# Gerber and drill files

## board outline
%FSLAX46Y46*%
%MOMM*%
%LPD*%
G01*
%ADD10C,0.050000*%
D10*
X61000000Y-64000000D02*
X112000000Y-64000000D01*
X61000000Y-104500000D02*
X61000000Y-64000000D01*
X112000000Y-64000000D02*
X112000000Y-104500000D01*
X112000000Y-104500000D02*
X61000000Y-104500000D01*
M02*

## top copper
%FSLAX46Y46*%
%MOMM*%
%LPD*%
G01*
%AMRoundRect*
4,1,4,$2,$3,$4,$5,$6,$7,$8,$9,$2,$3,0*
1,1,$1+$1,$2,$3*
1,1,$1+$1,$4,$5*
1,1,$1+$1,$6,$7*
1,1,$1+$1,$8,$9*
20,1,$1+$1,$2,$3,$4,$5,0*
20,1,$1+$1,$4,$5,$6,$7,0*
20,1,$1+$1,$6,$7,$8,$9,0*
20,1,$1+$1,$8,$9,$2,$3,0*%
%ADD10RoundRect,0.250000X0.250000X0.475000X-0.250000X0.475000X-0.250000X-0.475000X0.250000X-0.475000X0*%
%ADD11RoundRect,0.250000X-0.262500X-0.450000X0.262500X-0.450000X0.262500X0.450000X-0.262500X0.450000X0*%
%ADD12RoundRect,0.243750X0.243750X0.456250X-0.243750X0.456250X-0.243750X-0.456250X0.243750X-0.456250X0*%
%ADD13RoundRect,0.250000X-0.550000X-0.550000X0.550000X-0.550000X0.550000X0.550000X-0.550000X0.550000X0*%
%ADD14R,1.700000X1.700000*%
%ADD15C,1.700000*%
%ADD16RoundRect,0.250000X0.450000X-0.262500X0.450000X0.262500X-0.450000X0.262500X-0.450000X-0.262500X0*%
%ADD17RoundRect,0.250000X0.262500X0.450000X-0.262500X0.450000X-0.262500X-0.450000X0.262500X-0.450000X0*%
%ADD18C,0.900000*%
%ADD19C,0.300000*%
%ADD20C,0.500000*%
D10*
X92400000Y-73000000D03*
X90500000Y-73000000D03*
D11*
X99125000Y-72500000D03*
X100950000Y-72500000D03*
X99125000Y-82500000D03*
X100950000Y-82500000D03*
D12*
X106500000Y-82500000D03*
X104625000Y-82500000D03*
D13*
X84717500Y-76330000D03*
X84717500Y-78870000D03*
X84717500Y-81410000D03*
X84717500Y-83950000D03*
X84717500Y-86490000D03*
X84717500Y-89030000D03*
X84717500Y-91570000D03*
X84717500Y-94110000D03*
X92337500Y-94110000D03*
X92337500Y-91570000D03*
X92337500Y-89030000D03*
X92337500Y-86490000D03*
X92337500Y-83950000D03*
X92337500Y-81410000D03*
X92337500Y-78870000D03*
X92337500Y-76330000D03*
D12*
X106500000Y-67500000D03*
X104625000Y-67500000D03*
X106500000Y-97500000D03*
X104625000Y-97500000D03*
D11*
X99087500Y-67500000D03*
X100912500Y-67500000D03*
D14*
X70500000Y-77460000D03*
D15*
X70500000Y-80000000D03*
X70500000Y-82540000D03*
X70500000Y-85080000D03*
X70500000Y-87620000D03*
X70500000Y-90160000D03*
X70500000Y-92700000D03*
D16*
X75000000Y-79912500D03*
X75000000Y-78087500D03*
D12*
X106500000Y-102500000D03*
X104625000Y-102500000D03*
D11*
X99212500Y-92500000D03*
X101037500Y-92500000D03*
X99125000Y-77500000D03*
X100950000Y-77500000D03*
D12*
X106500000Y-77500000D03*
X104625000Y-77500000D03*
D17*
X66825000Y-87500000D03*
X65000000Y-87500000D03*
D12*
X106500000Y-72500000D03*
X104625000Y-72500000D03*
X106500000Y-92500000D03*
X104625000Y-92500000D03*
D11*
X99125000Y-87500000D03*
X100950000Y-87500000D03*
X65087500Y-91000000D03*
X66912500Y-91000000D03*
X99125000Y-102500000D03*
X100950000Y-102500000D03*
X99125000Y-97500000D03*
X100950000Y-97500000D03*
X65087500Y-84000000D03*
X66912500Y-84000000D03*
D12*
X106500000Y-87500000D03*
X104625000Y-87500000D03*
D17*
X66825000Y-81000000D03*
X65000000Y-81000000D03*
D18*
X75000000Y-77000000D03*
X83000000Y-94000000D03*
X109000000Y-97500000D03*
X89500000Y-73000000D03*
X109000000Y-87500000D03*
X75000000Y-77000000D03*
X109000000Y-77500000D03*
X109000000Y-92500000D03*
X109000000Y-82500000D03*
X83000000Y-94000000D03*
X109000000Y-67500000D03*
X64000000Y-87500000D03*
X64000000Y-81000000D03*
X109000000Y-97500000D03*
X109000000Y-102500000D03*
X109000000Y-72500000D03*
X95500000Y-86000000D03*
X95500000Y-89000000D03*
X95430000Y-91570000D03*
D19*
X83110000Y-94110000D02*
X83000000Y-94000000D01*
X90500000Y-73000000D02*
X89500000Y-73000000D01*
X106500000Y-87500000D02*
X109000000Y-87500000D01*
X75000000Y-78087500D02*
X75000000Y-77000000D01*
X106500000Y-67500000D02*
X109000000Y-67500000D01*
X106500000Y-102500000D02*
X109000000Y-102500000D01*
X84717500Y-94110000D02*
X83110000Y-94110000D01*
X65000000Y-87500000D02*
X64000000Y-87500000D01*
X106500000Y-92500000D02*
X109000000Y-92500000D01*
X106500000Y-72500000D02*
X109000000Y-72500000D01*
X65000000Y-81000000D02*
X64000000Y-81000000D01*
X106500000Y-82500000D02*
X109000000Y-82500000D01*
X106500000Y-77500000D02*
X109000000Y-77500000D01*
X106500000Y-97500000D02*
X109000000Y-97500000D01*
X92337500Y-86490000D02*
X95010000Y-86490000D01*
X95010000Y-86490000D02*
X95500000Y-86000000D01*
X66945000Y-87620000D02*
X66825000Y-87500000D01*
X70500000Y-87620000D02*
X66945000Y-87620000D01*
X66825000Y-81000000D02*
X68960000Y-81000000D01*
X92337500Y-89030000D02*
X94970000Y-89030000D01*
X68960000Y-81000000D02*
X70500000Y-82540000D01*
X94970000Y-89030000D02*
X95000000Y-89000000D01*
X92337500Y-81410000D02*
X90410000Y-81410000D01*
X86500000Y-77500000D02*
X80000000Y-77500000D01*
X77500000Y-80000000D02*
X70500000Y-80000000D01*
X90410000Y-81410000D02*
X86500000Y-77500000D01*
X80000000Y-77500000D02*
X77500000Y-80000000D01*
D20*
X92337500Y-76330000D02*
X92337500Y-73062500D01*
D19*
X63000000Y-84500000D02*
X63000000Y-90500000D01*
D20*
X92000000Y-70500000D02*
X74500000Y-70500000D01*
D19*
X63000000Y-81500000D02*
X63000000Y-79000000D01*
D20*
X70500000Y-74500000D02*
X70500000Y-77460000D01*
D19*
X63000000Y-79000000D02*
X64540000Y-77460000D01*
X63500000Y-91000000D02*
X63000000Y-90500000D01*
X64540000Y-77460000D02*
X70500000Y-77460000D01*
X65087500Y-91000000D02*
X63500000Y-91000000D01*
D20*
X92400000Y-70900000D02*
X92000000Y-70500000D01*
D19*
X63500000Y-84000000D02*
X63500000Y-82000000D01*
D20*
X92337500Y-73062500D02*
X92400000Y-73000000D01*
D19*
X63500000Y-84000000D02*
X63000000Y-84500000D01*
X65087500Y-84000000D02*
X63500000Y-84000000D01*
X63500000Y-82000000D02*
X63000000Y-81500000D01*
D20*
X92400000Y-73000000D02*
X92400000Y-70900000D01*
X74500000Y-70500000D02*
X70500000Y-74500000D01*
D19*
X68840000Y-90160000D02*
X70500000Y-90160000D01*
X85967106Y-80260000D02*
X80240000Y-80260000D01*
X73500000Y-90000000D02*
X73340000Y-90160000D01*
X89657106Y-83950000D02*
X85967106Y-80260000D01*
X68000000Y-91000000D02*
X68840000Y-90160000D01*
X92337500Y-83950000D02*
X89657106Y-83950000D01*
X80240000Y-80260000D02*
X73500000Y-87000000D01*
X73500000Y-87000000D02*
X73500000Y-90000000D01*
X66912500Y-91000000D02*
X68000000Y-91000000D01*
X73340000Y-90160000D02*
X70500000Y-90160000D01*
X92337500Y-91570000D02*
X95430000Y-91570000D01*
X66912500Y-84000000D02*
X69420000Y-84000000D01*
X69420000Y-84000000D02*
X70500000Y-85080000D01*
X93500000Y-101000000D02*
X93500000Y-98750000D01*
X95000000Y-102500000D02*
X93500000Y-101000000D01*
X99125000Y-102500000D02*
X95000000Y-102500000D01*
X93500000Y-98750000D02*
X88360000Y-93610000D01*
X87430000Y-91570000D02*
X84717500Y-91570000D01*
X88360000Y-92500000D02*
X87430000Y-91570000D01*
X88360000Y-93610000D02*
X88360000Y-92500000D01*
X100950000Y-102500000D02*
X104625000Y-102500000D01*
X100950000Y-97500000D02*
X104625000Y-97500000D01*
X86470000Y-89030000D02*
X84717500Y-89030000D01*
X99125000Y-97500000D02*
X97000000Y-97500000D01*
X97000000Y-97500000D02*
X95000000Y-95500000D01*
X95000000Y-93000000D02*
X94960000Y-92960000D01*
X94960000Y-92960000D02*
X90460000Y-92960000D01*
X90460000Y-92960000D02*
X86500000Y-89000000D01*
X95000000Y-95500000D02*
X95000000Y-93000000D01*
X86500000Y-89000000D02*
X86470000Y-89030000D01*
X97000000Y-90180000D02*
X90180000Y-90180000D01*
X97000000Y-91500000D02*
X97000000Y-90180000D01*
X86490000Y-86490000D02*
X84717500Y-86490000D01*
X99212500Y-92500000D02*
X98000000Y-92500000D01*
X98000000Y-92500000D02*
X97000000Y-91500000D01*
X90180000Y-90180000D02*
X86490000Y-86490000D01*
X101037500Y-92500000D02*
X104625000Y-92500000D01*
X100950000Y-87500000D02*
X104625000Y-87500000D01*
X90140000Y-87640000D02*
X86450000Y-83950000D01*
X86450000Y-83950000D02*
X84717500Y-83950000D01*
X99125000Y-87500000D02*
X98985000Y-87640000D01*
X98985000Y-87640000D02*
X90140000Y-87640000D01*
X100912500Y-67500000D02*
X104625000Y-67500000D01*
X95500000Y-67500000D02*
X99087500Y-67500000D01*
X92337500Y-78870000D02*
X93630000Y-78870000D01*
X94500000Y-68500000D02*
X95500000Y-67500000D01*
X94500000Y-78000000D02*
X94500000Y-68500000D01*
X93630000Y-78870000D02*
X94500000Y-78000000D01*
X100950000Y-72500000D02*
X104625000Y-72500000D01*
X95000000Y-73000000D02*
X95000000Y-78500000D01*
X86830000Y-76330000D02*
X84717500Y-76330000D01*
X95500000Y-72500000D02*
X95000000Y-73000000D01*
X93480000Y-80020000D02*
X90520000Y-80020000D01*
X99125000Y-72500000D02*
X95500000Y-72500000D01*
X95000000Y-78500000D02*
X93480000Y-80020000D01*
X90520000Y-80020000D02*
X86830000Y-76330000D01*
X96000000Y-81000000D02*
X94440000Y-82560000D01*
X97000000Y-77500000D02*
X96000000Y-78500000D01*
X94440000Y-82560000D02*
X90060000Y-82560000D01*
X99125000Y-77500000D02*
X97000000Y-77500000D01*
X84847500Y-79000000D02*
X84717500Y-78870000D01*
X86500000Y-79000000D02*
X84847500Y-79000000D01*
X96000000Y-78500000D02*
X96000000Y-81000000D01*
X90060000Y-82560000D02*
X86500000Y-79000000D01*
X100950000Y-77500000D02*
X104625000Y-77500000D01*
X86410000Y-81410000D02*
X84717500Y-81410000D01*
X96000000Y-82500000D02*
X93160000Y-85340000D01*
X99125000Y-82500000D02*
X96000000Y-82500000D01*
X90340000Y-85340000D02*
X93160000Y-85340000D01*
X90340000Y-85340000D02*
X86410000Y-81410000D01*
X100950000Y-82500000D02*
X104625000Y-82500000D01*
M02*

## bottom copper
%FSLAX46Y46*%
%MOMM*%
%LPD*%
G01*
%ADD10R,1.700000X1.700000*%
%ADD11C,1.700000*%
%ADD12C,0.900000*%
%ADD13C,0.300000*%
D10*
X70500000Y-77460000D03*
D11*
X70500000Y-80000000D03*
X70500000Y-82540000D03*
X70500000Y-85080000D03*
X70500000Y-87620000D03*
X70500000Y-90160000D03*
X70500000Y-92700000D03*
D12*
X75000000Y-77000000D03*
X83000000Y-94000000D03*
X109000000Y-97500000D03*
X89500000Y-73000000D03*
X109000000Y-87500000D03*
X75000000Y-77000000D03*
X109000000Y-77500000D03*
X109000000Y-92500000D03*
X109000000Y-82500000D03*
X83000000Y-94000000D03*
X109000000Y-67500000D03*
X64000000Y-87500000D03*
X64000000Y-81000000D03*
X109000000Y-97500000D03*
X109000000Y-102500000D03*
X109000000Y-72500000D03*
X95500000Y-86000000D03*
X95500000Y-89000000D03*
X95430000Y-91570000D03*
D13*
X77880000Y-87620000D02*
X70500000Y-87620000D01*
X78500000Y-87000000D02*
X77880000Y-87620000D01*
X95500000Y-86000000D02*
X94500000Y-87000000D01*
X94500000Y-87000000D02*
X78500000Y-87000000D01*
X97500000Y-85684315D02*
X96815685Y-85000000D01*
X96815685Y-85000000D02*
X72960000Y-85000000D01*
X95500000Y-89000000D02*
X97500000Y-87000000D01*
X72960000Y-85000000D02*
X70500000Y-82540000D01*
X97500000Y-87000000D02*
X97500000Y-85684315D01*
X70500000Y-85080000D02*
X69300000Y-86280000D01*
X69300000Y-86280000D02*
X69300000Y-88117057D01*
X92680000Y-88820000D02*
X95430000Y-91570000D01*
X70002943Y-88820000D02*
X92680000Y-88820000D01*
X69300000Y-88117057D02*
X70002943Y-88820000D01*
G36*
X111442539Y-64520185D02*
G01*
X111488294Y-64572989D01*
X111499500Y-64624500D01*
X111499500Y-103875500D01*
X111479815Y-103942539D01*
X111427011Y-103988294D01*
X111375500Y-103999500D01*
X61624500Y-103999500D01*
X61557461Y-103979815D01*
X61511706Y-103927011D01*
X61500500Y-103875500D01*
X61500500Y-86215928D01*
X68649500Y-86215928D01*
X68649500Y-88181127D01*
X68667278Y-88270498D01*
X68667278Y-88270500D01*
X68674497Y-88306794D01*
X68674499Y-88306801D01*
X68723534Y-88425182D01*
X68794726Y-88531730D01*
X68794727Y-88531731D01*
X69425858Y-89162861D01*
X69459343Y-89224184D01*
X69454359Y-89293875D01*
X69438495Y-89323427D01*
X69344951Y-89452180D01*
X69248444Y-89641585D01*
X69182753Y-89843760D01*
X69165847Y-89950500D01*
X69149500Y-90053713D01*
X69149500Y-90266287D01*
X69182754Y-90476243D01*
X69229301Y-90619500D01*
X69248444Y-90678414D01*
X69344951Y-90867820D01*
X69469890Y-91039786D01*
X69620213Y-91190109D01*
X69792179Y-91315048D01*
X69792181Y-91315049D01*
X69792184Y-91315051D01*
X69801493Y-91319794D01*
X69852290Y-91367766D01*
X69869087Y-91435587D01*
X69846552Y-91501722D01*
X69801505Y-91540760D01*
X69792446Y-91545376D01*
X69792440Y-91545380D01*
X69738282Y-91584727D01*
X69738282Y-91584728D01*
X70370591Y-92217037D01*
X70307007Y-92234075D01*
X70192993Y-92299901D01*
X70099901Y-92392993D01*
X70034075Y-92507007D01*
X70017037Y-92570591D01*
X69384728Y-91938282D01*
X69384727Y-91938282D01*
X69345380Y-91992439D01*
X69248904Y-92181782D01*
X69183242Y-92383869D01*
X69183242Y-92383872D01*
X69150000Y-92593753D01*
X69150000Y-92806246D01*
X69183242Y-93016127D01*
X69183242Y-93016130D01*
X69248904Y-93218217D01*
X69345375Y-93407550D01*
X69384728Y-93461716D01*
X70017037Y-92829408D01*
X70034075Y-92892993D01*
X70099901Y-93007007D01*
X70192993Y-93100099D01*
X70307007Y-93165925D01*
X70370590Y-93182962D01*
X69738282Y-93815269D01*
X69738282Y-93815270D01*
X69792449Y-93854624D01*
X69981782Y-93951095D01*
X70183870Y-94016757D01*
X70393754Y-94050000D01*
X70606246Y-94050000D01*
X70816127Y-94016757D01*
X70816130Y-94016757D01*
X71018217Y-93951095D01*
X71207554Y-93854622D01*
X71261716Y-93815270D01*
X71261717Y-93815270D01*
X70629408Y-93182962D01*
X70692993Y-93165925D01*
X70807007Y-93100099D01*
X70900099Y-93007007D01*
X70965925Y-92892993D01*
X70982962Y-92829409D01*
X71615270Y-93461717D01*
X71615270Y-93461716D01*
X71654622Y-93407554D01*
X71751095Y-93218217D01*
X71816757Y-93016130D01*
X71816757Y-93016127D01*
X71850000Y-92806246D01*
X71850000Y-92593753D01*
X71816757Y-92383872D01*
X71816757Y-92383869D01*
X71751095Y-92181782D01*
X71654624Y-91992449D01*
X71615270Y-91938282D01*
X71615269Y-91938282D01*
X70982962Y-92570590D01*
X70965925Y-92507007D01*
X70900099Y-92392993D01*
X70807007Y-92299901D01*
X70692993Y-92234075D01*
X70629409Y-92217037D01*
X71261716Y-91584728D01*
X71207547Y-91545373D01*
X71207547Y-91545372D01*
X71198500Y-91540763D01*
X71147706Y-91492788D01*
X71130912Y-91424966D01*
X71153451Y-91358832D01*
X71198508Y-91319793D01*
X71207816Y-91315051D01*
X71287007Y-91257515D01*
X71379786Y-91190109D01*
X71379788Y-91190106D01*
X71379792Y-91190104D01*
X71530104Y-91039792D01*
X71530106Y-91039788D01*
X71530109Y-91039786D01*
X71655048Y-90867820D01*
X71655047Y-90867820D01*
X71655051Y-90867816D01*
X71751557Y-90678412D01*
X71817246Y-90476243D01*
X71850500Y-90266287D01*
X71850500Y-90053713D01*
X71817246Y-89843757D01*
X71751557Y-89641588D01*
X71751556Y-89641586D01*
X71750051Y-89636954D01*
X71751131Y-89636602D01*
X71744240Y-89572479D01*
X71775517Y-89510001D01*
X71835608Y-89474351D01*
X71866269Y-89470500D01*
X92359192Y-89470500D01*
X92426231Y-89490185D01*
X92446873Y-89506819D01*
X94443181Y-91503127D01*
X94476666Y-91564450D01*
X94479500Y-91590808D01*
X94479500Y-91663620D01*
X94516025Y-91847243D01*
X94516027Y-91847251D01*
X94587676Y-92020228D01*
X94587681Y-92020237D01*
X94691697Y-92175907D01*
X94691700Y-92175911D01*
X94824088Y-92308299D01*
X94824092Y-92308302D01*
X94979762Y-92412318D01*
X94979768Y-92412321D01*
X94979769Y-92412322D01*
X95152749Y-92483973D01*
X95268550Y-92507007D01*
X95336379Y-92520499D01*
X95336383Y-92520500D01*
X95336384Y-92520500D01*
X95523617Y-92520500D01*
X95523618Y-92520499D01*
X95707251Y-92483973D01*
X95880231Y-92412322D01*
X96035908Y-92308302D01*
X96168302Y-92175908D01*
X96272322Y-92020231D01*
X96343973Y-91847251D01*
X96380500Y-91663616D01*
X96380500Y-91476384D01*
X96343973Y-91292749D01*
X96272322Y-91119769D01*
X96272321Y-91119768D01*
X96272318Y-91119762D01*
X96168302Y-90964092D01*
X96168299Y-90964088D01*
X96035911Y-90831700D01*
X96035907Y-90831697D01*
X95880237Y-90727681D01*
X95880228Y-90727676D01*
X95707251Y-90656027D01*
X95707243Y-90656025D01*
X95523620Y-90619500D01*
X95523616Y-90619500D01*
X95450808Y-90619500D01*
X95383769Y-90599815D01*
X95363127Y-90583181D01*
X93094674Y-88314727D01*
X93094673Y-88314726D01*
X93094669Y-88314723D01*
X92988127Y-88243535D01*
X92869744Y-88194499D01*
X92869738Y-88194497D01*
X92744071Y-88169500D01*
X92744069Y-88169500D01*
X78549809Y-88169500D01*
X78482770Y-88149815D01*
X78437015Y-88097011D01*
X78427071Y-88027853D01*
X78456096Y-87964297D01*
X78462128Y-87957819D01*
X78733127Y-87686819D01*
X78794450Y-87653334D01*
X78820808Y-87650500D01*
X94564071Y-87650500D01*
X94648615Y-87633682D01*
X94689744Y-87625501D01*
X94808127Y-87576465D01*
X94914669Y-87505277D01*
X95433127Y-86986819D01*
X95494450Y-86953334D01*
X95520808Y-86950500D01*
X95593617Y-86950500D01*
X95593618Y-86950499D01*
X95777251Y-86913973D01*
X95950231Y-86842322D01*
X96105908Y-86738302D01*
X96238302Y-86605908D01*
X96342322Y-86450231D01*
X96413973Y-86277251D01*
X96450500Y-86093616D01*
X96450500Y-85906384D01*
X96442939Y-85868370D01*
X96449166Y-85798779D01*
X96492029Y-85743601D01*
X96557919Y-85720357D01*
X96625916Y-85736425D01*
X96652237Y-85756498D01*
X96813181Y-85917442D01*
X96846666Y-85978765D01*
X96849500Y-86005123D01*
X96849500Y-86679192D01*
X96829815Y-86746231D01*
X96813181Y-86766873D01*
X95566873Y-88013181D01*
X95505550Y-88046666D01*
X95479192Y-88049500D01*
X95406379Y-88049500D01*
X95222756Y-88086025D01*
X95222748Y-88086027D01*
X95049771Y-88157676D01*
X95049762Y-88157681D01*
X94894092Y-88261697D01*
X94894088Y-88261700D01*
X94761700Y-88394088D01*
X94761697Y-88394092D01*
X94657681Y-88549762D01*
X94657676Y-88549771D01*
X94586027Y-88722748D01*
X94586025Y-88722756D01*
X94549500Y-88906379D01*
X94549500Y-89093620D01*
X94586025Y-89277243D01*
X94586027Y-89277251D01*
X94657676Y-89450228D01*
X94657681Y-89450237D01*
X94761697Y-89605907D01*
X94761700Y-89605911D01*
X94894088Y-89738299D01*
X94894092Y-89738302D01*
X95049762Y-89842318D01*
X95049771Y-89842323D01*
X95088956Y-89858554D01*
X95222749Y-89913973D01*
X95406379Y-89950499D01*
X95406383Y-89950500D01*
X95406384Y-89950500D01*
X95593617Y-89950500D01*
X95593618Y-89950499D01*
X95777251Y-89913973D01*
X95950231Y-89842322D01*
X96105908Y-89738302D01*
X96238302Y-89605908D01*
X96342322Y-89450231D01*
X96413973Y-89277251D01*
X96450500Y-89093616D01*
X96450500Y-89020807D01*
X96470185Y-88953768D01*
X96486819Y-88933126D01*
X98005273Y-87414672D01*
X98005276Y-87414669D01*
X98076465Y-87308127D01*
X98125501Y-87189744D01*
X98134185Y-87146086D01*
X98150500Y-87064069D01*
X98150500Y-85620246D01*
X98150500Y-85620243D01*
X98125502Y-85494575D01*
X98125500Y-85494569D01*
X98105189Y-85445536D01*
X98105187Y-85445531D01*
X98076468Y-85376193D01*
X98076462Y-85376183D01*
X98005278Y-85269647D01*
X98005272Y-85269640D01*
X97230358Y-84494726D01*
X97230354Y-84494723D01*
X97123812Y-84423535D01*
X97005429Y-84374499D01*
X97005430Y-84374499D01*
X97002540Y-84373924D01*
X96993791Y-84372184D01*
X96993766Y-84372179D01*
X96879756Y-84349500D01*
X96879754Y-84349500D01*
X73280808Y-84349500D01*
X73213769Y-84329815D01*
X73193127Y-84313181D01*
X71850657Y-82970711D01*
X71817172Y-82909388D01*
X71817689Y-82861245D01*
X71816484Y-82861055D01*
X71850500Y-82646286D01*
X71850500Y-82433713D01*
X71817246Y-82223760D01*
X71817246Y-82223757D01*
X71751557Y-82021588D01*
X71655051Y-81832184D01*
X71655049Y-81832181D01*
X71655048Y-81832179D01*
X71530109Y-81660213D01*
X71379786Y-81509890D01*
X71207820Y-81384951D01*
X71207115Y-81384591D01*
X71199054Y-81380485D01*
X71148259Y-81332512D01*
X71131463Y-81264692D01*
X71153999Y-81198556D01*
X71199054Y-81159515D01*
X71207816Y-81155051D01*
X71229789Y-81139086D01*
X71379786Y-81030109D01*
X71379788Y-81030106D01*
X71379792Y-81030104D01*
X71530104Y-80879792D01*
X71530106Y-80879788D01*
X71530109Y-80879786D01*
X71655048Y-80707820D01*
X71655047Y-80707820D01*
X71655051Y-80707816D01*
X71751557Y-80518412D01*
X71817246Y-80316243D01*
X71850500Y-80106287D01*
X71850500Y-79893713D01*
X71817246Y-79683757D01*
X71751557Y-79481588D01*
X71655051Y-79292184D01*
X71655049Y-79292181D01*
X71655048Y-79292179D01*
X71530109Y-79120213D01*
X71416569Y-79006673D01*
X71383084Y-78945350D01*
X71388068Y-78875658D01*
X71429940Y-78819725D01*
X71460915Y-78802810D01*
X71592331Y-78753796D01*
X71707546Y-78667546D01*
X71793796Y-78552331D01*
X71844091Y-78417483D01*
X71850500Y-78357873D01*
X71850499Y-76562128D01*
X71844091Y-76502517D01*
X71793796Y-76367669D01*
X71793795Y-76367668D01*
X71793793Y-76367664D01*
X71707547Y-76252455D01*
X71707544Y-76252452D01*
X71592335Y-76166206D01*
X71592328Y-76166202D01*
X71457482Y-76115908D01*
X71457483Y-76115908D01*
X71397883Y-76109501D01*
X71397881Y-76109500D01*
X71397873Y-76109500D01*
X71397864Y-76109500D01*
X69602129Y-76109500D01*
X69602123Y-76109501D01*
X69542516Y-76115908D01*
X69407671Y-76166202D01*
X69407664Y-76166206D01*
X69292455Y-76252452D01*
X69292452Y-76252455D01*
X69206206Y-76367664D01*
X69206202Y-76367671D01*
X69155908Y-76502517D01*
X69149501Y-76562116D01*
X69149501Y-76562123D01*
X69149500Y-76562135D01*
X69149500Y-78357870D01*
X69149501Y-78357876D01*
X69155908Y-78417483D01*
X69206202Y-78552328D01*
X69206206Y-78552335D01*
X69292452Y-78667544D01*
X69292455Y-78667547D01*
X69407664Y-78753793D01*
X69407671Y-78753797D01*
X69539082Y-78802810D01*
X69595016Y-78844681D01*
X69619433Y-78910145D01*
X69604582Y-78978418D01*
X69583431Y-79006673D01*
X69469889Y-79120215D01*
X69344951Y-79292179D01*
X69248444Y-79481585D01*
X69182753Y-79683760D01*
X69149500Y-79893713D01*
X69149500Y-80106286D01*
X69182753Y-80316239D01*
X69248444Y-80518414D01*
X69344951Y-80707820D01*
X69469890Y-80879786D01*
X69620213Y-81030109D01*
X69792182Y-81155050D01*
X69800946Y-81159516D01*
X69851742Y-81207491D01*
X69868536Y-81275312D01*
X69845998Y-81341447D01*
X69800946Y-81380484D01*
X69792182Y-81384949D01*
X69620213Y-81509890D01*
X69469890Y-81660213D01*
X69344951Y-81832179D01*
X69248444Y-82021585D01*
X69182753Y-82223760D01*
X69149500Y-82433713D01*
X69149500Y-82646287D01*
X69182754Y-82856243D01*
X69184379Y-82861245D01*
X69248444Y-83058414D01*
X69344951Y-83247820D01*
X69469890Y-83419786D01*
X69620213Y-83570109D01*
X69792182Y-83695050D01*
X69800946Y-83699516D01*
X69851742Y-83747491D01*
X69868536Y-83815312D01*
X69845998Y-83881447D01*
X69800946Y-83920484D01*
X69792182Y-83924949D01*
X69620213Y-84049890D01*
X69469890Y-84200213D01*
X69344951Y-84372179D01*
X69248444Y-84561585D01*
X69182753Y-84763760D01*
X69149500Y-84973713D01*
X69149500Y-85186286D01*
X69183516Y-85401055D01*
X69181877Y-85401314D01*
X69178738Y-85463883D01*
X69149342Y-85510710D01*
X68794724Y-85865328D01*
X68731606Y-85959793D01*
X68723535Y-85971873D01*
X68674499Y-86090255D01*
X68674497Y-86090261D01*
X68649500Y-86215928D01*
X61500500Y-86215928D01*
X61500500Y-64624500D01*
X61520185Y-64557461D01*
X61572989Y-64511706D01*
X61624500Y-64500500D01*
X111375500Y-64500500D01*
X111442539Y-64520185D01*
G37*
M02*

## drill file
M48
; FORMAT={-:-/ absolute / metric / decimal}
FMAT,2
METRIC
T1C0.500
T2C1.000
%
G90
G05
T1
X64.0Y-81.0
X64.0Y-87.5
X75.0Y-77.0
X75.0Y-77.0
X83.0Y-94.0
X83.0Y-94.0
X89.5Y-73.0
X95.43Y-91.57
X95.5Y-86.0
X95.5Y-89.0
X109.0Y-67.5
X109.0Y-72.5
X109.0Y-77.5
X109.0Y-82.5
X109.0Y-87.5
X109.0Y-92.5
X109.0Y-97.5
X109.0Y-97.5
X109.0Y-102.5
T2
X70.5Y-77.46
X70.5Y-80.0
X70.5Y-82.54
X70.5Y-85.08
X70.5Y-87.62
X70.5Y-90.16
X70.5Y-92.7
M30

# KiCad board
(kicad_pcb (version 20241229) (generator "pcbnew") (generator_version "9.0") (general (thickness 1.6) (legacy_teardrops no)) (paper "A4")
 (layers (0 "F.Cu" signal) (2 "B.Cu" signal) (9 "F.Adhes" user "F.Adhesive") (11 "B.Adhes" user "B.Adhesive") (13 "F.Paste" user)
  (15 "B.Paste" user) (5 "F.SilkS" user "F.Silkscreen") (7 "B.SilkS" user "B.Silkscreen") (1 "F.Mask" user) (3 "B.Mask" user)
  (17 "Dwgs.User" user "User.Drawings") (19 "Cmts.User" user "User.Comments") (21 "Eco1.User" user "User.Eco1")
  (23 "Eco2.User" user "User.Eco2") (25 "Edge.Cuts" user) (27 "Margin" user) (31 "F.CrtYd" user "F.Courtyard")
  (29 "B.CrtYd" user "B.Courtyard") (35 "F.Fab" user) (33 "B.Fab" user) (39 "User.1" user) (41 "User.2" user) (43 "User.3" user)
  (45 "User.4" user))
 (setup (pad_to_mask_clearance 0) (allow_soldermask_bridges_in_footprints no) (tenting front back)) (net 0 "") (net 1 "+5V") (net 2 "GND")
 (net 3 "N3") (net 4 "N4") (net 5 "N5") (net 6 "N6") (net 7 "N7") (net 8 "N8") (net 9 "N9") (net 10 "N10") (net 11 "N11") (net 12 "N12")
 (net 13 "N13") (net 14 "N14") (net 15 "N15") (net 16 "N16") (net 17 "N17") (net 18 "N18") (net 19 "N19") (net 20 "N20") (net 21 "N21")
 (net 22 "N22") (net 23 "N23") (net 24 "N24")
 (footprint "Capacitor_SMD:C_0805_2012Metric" (layer "F.Cu") (at 91.45 73 180)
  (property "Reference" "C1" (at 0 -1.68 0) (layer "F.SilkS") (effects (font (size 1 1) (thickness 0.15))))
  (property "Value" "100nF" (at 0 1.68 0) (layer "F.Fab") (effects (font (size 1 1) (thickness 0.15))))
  (pad "1" smd roundrect (at -0.95 0 180) (size 1 1.45) (layers "F.Cu" "F.Mask" "F.Paste") (roundrect_rratio 0.25) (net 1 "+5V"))
  (pad "2" smd roundrect (at 0.95 0 180) (size 1 1.45) (layers "F.Cu" "F.Mask" "F.Paste") (roundrect_rratio 0.25) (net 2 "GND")))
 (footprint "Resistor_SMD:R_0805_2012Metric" (layer "F.Cu") (at 100.0375 72.5)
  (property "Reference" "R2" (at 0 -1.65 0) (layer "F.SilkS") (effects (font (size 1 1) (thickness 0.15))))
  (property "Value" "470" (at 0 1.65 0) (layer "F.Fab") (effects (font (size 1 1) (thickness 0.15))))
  (pad "1" smd roundrect (at -0.9125 0) (size 1.025 1.4) (layers "F.Cu" "F.Mask" "F.Paste") (roundrect_rratio 0.243902) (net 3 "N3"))
  (pad "2" smd roundrect (at 0.9125 0) (size 1.025 1.4) (layers "F.Cu" "F.Mask" "F.Paste") (roundrect_rratio 0.243902) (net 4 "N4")))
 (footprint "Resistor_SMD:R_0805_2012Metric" (layer "F.Cu") (at 100.0375 82.5)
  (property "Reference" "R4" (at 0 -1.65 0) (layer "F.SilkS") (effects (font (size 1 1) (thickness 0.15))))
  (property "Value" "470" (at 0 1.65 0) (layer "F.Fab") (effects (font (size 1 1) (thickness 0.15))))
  (pad "1" smd roundrect (at -0.9125 0) (size 1.025 1.4) (layers "F.Cu" "F.Mask" "F.Paste") (roundrect_rratio 0.243902) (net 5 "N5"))
  (pad "2" smd roundrect (at 0.9125 0) (size 1.025 1.4) (layers "F.Cu" "F.Mask" "F.Paste") (roundrect_rratio 0.243902) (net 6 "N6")))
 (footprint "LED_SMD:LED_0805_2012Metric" (layer "F.Cu") (at 105.5625 82.5 180)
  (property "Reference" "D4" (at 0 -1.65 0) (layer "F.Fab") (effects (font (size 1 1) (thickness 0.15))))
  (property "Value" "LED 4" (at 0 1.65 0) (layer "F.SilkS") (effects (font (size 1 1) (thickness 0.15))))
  (pad "1" smd roundrect (at -0.9375 0 180) (size 0.975 1.4) (layers "F.Cu" "F.Mask" "F.Paste") (roundrect_rratio 0.25) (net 2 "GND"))
  (pad "2" smd roundrect (at 0.9375 0 180) (size 0.975 1.4) (layers "F.Cu" "F.Mask" "F.Paste") (roundrect_rratio 0.25) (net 6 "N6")))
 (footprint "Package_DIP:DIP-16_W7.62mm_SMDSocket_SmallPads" (layer "F.Cu") (at 88.5275 85.22)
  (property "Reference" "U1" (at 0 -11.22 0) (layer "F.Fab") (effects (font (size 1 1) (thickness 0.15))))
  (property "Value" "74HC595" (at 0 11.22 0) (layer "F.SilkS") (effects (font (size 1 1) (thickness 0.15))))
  (pad "1" smd roundrect (at -3.81 -8.89) (size 1.6 1.6) (layers "F.Cu" "F.Mask" "F.Paste") (roundrect_rratio 0.15625) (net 3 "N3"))
  (pad "2" smd roundrect (at -3.81 -6.35) (size 1.6 1.6) (layers "F.Cu" "F.Mask" "F.Paste") (roundrect_rratio 0.15625) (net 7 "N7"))
  (pad "3" smd roundrect (at -3.81 -3.81) (size 1.6 1.6) (layers "F.Cu" "F.Mask" "F.Paste") (roundrect_rratio 0.15625) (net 5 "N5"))
  (pad "4" smd roundrect (at -3.81 -1.27) (size 1.6 1.6) (layers "F.Cu" "F.Mask" "F.Paste") (roundrect_rratio 0.15625) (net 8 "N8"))
  (pad "5" smd roundrect (at -3.81 1.27) (size 1.6 1.6) (layers "F.Cu" "F.Mask" "F.Paste") (roundrect_rratio 0.15625) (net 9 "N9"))
  (pad "6" smd roundrect (at -3.81 3.81) (size 1.6 1.6) (layers "F.Cu" "F.Mask" "F.Paste") (roundrect_rratio 0.15625) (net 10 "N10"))
  (pad "7" smd roundrect (at -3.81 6.35) (size 1.6 1.6) (layers "F.Cu" "F.Mask" "F.Paste") (roundrect_rratio 0.15625) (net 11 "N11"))
  (pad "8" smd roundrect (at -3.81 8.89) (size 1.6 1.6) (layers "F.Cu" "F.Mask" "F.Paste") (roundrect_rratio 0.15625) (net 2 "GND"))
  (pad "9" smd roundrect (at 3.81 8.89) (size 1.6 1.6) (layers "F.Cu" "F.Mask" "F.Paste") (roundrect_rratio 0.15625) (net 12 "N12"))
  (pad "10" smd roundrect (at 3.81 6.35) (size 1.6 1.6) (layers "F.Cu" "F.Mask" "F.Paste") (roundrect_rratio 0.15625) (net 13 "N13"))
  (pad "11" smd roundrect (at 3.81 3.81) (size 1.6 1.6) (layers "F.Cu" "F.Mask" "F.Paste") (roundrect_rratio 0.15625) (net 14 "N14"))
  (pad "12" smd roundrect (at 3.81 1.27) (size 1.6 1.6) (layers "F.Cu" "F.Mask" "F.Paste") (roundrect_rratio 0.15625) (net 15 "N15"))
  (pad "13" smd roundrect (at 3.81 -1.27) (size 1.6 1.6) (layers "F.Cu" "F.Mask" "F.Paste") (roundrect_rratio 0.15625) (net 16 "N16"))
  (pad "14" smd roundrect (at 3.81 -3.81) (size 1.6 1.6) (layers "F.Cu" "F.Mask" "F.Paste") (roundrect_rratio 0.15625) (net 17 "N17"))
  (pad "15" smd roundrect (at 3.81 -6.35) (size 1.6 1.6) (layers "F.Cu" "F.Mask" "F.Paste") (roundrect_rratio 0.15625) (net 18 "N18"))
  (pad "16" smd roundrect (at 3.81 -8.89) (size 1.6 1.6) (layers "F.Cu" "F.Mask" "F.Paste") (roundrect_rratio 0.15625) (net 1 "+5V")))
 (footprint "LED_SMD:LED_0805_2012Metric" (layer "F.Cu") (at 105.5625 67.5 180)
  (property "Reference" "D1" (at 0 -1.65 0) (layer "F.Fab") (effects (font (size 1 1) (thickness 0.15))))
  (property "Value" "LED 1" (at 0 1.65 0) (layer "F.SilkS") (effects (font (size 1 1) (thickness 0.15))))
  (pad "1" smd roundrect (at -0.9375 0 180) (size 0.975 1.4) (layers "F.Cu" "F.Mask" "F.Paste") (roundrect_rratio 0.25) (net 2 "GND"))
  (pad "2" smd roundrect (at 0.9375 0 180) (size 0.975 1.4) (layers "F.Cu" "F.Mask" "F.Paste") (roundrect_rratio 0.25) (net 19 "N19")))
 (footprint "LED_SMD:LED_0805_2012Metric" (layer "F.Cu") (at 105.5625 97.5 180)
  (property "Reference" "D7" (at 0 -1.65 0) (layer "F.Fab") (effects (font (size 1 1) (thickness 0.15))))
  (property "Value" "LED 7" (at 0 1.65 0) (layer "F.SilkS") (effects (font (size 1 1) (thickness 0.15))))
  (pad "1" smd roundrect (at -0.9375 0 180) (size 0.975 1.4) (layers "F.Cu" "F.Mask" "F.Paste") (roundrect_rratio 0.25) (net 2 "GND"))
  (pad "2" smd roundrect (at 0.9375 0 180) (size 0.975 1.4) (layers "F.Cu" "F.Mask" "F.Paste") (roundrect_rratio 0.25) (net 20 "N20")))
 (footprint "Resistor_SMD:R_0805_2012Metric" (layer "F.Cu") (at 100 67.5)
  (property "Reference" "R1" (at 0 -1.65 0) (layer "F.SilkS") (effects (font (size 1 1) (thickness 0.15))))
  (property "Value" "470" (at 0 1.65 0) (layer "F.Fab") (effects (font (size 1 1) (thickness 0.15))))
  (pad "1" smd roundrect (at -0.9125 0) (size 1.025 1.4) (layers "F.Cu" "F.Mask" "F.Paste") (roundrect_rratio 0.243902) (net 18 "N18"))
  (pad "2" smd roundrect (at 0.9125 0) (size 1.025 1.4) (layers "F.Cu" "F.Mask" "F.Paste") (roundrect_rratio 0.243902) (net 19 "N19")))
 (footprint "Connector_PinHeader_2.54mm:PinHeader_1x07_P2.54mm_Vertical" (layer "F.Cu") (at 70.5 77.46)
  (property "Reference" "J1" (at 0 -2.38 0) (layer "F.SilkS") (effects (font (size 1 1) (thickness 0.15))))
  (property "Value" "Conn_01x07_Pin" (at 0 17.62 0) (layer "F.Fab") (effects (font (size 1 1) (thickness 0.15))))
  (pad "1" thru_hole rect (at 0 0) (size 1.7 1.7) (drill 1) (layers "*.Cu" "*.Mask") (remove_unused_layers no) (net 1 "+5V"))
  (pad "2" thru_hole circle (at 0 2.54) (size 1.7 1.7) (drill 1) (layers "*.Cu" "*.Mask") (remove_unused_layers no) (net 17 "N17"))
  (pad "3" thru_hole circle (at 0 5.08) (size 1.7 1.7) (drill 1) (layers "*.Cu" "*.Mask") (remove_unused_layers no) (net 14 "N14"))
  (pad "4" thru_hole circle (at 0 7.62) (size 1.7 1.7) (drill 1) (layers "*.Cu" "*.Mask") (remove_unused_layers no) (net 13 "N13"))
  (pad "5" thru_hole circle (at 0 10.16) (size 1.7 1.7) (drill 1) (layers "*.Cu" "*.Mask") (remove_unused_layers no) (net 15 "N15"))
  (pad "6" thru_hole circle (at 0 12.7) (size 1.7 1.7) (drill 1) (layers "*.Cu" "*.Mask") (remove_unused_layers no) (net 16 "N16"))
  (pad "7" thru_hole circle (at 0 15.24) (size 1.7 1.7) (drill 1) (layers "*.Cu" "*.Mask") (remove_unused_layers no) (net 2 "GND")))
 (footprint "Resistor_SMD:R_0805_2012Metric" (layer "F.Cu") (at 75 79 90)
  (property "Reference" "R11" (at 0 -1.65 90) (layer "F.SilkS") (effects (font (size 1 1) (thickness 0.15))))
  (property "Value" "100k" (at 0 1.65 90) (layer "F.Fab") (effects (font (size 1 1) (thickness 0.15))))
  (pad "1" smd roundrect (at -0.9125 0 90) (size 1.025 1.4) (layers "F.Cu" "F.Mask" "F.Paste") (roundrect_rratio 0.243902) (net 17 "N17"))
  (pad "2" smd roundrect (at 0.9125 0 90) (size 1.025 1.4) (layers "F.Cu" "F.Mask" "F.Paste") (roundrect_rratio 0.243902) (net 2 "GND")))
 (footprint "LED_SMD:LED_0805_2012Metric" (layer "F.Cu") (at 105.5625 102.5 180)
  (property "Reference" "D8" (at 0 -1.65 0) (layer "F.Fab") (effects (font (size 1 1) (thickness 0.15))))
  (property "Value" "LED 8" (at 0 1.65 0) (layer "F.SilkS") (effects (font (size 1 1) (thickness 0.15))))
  (pad "1" smd roundrect (at -0.9375 0 180) (size 0.975 1.4) (layers "F.Cu" "F.Mask" "F.Paste") (roundrect_rratio 0.25) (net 2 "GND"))
  (pad "2" smd roundrect (at 0.9375 0 180) (size 0.975 1.4) (layers "F.Cu" "F.Mask" "F.Paste") (roundrect_rratio 0.25) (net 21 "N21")))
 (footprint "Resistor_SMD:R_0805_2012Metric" (layer "F.Cu") (at 100.125 92.5)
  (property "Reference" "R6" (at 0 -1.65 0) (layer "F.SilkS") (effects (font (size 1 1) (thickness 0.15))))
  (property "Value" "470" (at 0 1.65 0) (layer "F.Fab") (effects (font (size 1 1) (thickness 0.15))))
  (pad "1" smd roundrect (at -0.9125 0) (size 1.025 1.4) (layers "F.Cu" "F.Mask" "F.Paste") (roundrect_rratio 0.243902) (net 9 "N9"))
  (pad "2" smd roundrect (at 0.9125 0) (size 1.025 1.4) (layers "F.Cu" "F.Mask" "F.Paste") (roundrect_rratio 0.243902) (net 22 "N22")))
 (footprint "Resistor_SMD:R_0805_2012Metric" (layer "F.Cu") (at 100.0375 77.5)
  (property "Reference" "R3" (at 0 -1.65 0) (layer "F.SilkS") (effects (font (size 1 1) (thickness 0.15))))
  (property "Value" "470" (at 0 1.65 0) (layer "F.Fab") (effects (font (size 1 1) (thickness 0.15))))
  (pad "1" smd roundrect (at -0.9125 0) (size 1.025 1.4) (layers "F.Cu" "F.Mask" "F.Paste") (roundrect_rratio 0.243902) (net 7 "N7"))
  (pad "2" smd roundrect (at 0.9125 0) (size 1.025 1.4) (layers "F.Cu" "F.Mask" "F.Paste") (roundrect_rratio 0.243902) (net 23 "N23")))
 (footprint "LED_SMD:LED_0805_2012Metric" (layer "F.Cu") (at 105.5625 77.5 180)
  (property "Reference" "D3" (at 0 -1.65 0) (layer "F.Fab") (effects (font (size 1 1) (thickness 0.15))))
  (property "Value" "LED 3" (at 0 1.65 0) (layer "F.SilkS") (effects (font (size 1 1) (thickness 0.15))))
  (pad "1" smd roundrect (at -0.9375 0 180) (size 0.975 1.4) (layers "F.Cu" "F.Mask" "F.Paste") (roundrect_rratio 0.25) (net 2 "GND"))
  (pad "2" smd roundrect (at 0.9375 0 180) (size 0.975 1.4) (layers "F.Cu" "F.Mask" "F.Paste") (roundrect_rratio 0.25) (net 23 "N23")))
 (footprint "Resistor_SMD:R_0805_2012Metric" (layer "F.Cu") (at 65.9125 87.5 180)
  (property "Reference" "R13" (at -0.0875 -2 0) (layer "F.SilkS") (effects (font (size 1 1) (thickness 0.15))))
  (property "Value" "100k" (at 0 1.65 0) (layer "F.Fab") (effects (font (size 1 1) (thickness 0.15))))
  (pad "1" smd roundrect (at -0.9125 0 180) (size 1.025 1.4) (layers "F.Cu" "F.Mask" "F.Paste") (roundrect_rratio 0.243902) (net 15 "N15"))
  (pad "2" smd roundrect (at 0.9125 0 180) (size 1.025 1.4) (layers "F.Cu" "F.Mask" "F.Paste") (roundrect_rratio 0.243902) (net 2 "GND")))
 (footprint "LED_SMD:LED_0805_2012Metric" (layer "F.Cu") (at 105.5625 72.5 180)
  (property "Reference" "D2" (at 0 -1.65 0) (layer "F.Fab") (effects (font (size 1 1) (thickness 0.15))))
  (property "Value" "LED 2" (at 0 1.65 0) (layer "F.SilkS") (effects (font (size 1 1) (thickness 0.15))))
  (pad "1" smd roundrect (at -0.9375 0 180) (size 0.975 1.4) (layers "F.Cu" "F.Mask" "F.Paste") (roundrect_rratio 0.25) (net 2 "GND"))
  (pad "2" smd roundrect (at 0.9375 0 180) (size 0.975 1.4) (layers "F.Cu" "F.Mask" "F.Paste") (roundrect_rratio 0.25) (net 4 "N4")))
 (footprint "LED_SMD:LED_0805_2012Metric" (layer "F.Cu") (at 105.5625 92.5 180)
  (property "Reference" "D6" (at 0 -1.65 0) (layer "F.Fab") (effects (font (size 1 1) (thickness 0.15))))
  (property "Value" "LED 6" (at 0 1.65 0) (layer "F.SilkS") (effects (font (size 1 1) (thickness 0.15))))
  (pad "1" smd roundrect (at -0.9375 0 180) (size 0.975 1.4) (layers "F.Cu" "F.Mask" "F.Paste") (roundrect_rratio 0.25) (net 2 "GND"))
  (pad "2" smd roundrect (at 0.9375 0 180) (size 0.975 1.4) (layers "F.Cu" "F.Mask" "F.Paste") (roundrect_rratio 0.25) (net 22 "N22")))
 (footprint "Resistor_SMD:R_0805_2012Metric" (layer "F.Cu") (at 100.0375 87.5)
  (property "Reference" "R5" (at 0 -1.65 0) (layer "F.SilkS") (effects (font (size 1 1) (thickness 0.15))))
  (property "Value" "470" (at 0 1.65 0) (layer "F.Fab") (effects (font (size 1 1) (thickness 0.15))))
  (pad "1" smd roundrect (at -0.9125 0) (size 1.025 1.4) (layers "F.Cu" "F.Mask" "F.Paste") (roundrect_rratio 0.243902) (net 8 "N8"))
  (pad "2" smd roundrect (at 0.9125 0) (size 1.025 1.4) (layers "F.Cu" "F.Mask" "F.Paste") (roundrect_rratio 0.243902) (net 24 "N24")))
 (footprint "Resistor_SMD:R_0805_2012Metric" (layer "F.Cu") (at 66 91)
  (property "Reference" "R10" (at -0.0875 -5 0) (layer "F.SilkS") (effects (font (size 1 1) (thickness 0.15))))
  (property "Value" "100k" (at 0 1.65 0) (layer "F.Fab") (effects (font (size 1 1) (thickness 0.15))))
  (pad "1" smd roundrect (at -0.9125 0) (size 1.025 1.4) (layers "F.Cu" "F.Mask" "F.Paste") (roundrect_rratio 0.243902) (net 1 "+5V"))
  (pad "2" smd roundrect (at 0.9125 0) (size 1.025 1.4) (layers "F.Cu" "F.Mask" "F.Paste") (roundrect_rratio 0.243902) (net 16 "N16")))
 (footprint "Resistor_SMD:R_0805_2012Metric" (layer "F.Cu") (at 100.0375 102.5)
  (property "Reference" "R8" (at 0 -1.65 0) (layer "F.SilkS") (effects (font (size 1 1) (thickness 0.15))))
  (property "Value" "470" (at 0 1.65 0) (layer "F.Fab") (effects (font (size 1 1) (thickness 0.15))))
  (pad "1" smd roundrect (at -0.9125 0) (size 1.025 1.4) (layers "F.Cu" "F.Mask" "F.Paste") (roundrect_rratio 0.243902) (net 11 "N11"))
  (pad "2" smd roundrect (at 0.9125 0) (size 1.025 1.4) (layers "F.Cu" "F.Mask" "F.Paste") (roundrect_rratio 0.243902) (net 21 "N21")))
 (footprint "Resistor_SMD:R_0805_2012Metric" (layer "F.Cu") (at 100.0375 97.5)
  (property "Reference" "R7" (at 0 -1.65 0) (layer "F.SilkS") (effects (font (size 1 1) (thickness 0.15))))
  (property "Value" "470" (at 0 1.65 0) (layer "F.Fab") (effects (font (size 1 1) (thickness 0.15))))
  (pad "1" smd roundrect (at -0.9125 0) (size 1.025 1.4) (layers "F.Cu" "F.Mask" "F.Paste") (roundrect_rratio 0.243902) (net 10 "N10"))
  (pad "2" smd roundrect (at 0.9125 0) (size 1.025 1.4) (layers "F.Cu" "F.Mask" "F.Paste") (roundrect_rratio 0.243902) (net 20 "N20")))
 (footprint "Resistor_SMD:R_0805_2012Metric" (layer "F.Cu") (at 66 84)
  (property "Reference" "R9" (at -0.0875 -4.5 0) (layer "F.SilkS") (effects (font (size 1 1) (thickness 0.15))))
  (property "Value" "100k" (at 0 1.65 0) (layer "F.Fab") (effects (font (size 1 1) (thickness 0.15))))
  (pad "1" smd roundrect (at -0.9125 0) (size 1.025 1.4) (layers "F.Cu" "F.Mask" "F.Paste") (roundrect_rratio 0.243902) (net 1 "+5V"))
  (pad "2" smd roundrect (at 0.9125 0) (size 1.025 1.4) (layers "F.Cu" "F.Mask" "F.Paste") (roundrect_rratio 0.243902) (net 13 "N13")))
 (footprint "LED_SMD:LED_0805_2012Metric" (layer "F.Cu") (at 105.5625 87.5 180)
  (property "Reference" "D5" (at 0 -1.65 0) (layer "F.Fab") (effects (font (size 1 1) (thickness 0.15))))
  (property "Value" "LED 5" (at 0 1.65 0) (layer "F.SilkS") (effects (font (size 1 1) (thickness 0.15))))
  (pad "1" smd roundrect (at -0.9375 0 180) (size 0.975 1.4) (layers "F.Cu" "F.Mask" "F.Paste") (roundrect_rratio 0.25) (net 2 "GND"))
  (pad "2" smd roundrect (at 0.9375 0 180) (size 0.975 1.4) (layers "F.Cu" "F.Mask" "F.Paste") (roundrect_rratio 0.25) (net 24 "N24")))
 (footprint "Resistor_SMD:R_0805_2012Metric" (layer "F.Cu") (at 65.9125 81 180)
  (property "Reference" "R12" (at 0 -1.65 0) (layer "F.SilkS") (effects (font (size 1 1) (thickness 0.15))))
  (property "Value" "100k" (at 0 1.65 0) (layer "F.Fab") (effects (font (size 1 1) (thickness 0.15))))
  (pad "1" smd roundrect (at -0.9125 0 180) (size 1.025 1.4) (layers "F.Cu" "F.Mask" "F.Paste") (roundrect_rratio 0.243902) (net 14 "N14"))
  (pad "2" smd roundrect (at 0.9125 0 180) (size 1.025 1.4) (layers "F.Cu" "F.Mask" "F.Paste") (roundrect_rratio 0.243902) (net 2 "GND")))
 (gr_line (start 61 64) (end 112 64) (stroke (width 0.05) (type default)) (layer "Edge.Cuts"))
 (gr_line (start 61 104.5) (end 61 64) (stroke (width 0.05) (type default)) (layer "Edge.Cuts"))
 (gr_line (start 112 64) (end 112 104.5) (stroke (width 0.05) (type default)) (layer "Edge.Cuts"))
 (gr_line (start 112 104.5) (end 61 104.5) (stroke (width 0.05) (type default)) (layer "Edge.Cuts"))
 (segment (start 83.11 94.11) (end 83 94) (width 0.3) (layer "F.Cu") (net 2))
 (segment (start 90.5 73) (end 89.5 73) (width 0.3) (layer "F.Cu") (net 2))
 (segment (start 106.5 87.5) (end 109 87.5) (width 0.3) (layer "F.Cu") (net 2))
 (segment (start 75 78.0875) (end 75 77) (width 0.3) (layer "F.Cu") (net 2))
 (segment (start 106.5 67.5) (end 109 67.5) (width 0.3) (layer "F.Cu") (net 2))
 (segment (start 106.5 102.5) (end 109 102.5) (width 0.3) (layer "F.Cu") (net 2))
 (segment (start 84.7175 94.11) (end 83.11 94.11) (width 0.3) (layer "F.Cu") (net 2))
 (segment (start 65 87.5) (end 64 87.5) (width 0.3) (layer "F.Cu") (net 2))
 (segment (start 106.5 92.5) (end 109 92.5) (width 0.3) (layer "F.Cu") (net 2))
 (segment (start 106.5 72.5) (end 109 72.5) (width 0.3) (layer "F.Cu") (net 2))
 (segment (start 65 81) (end 64 81) (width 0.3) (layer "F.Cu") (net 2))
 (segment (start 106.5 82.5) (end 109 82.5) (width 0.3) (layer "F.Cu") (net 2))
 (segment (start 106.5 77.5) (end 109 77.5) (width 0.3) (layer "F.Cu") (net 2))
 (segment (start 106.5 97.5) (end 109 97.5) (width 0.3) (layer "F.Cu") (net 2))
 (via (at 75 77) (size 0.9) (drill 0.5) (layers "F.Cu" "B.Cu") (free yes) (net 2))
 (via (at 83 94) (size 0.9) (drill 0.5) (layers "F.Cu" "B.Cu") (free yes) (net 2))
 (via (at 109 97.5) (size 0.9) (drill 0.5) (layers "F.Cu" "B.Cu") (free yes) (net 2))
 (via (at 89.5 73) (size 0.9) (drill 0.5) (layers "F.Cu" "B.Cu") (free yes) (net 2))
 (via (at 109 87.5) (size 0.9) (drill 0.5) (layers "F.Cu" "B.Cu") (free yes) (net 2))
 (via (at 75 77) (size 0.9) (drill 0.5) (layers "F.Cu" "B.Cu") (free yes) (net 2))
 (via (at 109 77.5) (size 0.9) (drill 0.5) (layers "F.Cu" "B.Cu") (free yes) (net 2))
 (via (at 109 92.5) (size 0.9) (drill 0.5) (layers "F.Cu" "B.Cu") (free yes) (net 2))
 (via (at 109 82.5) (size 0.9) (drill 0.5) (layers "F.Cu" "B.Cu") (free yes) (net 2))
 (via (at 83 94) (size 0.9) (drill 0.5) (layers "F.Cu" "B.Cu") (free yes) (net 2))
 (via (at 109 67.5) (size 0.9) (drill 0.5) (layers "F.Cu" "B.Cu") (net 2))
 (via (at 64 87.5) (size 0.9) (drill 0.5) (layers "F.Cu" "B.Cu") (free yes) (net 2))
 (via (at 64 81) (size 0.9) (drill 0.5) (layers "F.Cu" "B.Cu") (free yes) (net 2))
 (via (at 109 97.5) (size 0.9) (drill 0.5) (layers "F.Cu" "B.Cu") (free yes) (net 2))
 (via (at 109 102.5) (size 0.9) (drill 0.5) (layers "F.Cu" "B.Cu") (free yes) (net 2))
 (via (at 109 72.5) (size 0.9) (drill 0.5) (layers "F.Cu" "B.Cu") (free yes) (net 2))
 (segment (start 92.3375 86.49) (end 95.01 86.49) (width 0.3) (layer "F.Cu") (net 15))
 (segment (start 95.01 86.49) (end 95.5 86) (width 0.3) (layer "F.Cu") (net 15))
 (segment (start 66.945 87.62) (end 66.825 87.5) (width 0.3) (layer "F.Cu") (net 15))
 (segment (start 70.5 87.62) (end 66.945 87.62) (width 0.3) (layer "F.Cu") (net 15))
 (via (at 95.5 86) (size 0.9) (drill 0.5) (layers "F.Cu" "B.Cu") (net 15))
 (segment (start 77.88 87.62) (end 70.5 87.62) (width 0.3) (layer "B.Cu") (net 15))
 (segment (start 78.5 87) (end 77.88 87.62) (width 0.3) (layer "B.Cu") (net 15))
 (segment (start 95.5 86) (end 94.5 87) (width 0.3) (layer "B.Cu") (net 15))
 (segment (start 94.5 87) (end 78.5 87) (width 0.3) (layer "B.Cu") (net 15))
 (segment (start 66.825 81) (end 68.96 81) (width 0.3) (layer "F.Cu") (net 14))
 (segment (start 92.3375 89.03) (end 94.97 89.03) (width 0.3) (layer "F.Cu") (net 14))
 (segment (start 68.96 81) (end 70.5 82.54) (width 0.3) (layer "F.Cu") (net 14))
 (segment (start 94.97 89.03) (end 95 89) (width 0.3) (layer "F.Cu") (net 14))
 (via (at 95.5 89) (size 0.9) (drill 0.5) (layers "F.Cu" "B.Cu") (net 14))
 (segment (start 97.5 85.684315) (end 96.815685 85) (width 0.3) (layer "B.Cu") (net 14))
 (segment (start 96.815685 85) (end 72.96 85) (width 0.3) (layer "B.Cu") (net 14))
 (segment (start 95.5 89) (end 97.5 87) (width 0.3) (layer "B.Cu") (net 14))
 (segment (start 72.96 85) (end 70.5 82.54) (width 0.3) (layer "B.Cu") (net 14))
 (segment (start 97.5 87) (end 97.5 85.684315) (width 0.3) (layer "B.Cu") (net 14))
 (segment (start 92.3375 81.41) (end 90.41 81.41) (width 0.3) (layer "F.Cu") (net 17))
 (segment (start 86.5 77.5) (end 80 77.5) (width 0.3) (layer "F.Cu") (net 17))
 (segment (start 77.5 80) (end 70.5 80) (width 0.3) (layer "F.Cu") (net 17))
 (segment (start 90.41 81.41) (end 86.5 77.5) (width 0.3) (layer "F.Cu") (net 17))
 (segment (start 80 77.5) (end 77.5 80) (width 0.3) (layer "F.Cu") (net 17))
 (segment (start 92.3375 76.33) (end 92.3375 73.0625) (width 0.5) (layer "F.Cu") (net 1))
 (segment (start 63 84.5) (end 63 90.5) (width 0.3) (layer "F.Cu") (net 1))
 (segment (start 92 70.5) (end 74.5 70.5) (width 0.5) (layer "F.Cu") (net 1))
 (segment (start 63 81.5) (end 63 79) (width 0.3) (layer "F.Cu") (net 1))
 (segment (start 70.5 74.5) (end 70.5 77.46) (width 0.5) (layer "F.Cu") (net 1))
 (segment (start 63 79) (end 64.54 77.46) (width 0.3) (layer "F.Cu") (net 1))
 (segment (start 63.5 91) (end 63 90.5) (width 0.3) (layer "F.Cu") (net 1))
 (segment (start 64.54 77.46) (end 70.5 77.46) (width 0.3) (layer "F.Cu") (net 1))
 (segment (start 65.0875 91) (end 63.5 91) (width 0.3) (layer "F.Cu") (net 1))
 (segment (start 92.4 70.9) (end 92 70.5) (width 0.5) (layer "F.Cu") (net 1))
 (segment (start 63.5 84) (end 63.5 82) (width 0.3) (layer "F.Cu") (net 1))
 (segment (start 92.3375 73.0625) (end 92.4 73) (width 0.5) (layer "F.Cu") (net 1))
 (segment (start 63.5 84) (end 63 84.5) (width 0.3) (layer "F.Cu") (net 1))
 (segment (start 65.0875 84) (end 63.5 84) (width 0.3) (layer "F.Cu") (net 1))
 (segment (start 63.5 82) (end 63 81.5) (width 0.3) (layer "F.Cu") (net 1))
 (segment (start 92.4 73) (end 92.4 70.9) (width 0.5) (layer "F.Cu") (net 1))
 (segment (start 74.5 70.5) (end 70.5 74.5) (width 0.5) (layer "F.Cu") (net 1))
 (segment (start 68.84 90.16) (end 70.5 90.16) (width 0.3) (layer "F.Cu") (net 16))
 (segment (start 85.967106 80.26) (end 80.24 80.26) (width 0.3) (layer "F.Cu") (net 16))
 (segment (start 73.5 90) (end 73.34 90.16) (width 0.3) (layer "F.Cu") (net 16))
 (segment (start 89.657106 83.95) (end 85.967106 80.26) (width 0.3) (layer "F.Cu") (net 16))
 (segment (start 68 91) (end 68.84 90.16) (width 0.3) (layer "F.Cu") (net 16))
 (segment (start 92.3375 83.95) (end 89.657106 83.95) (width 0.3) (layer "F.Cu") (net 16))
 (segment (start 80.24 80.26) (end 73.5 87) (width 0.3) (layer "F.Cu") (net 16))
 (segment (start 73.5 87) (end 73.5 90) (width 0.3) (layer "F.Cu") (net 16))
 (segment (start 66.9125 91) (end 68 91) (width 0.3) (layer "F.Cu") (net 16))
 (segment (start 73.34 90.16) (end 70.5 90.16) (width 0.3) (layer "F.Cu") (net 16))
 (segment (start 92.3375 91.57) (end 95.43 91.57) (width 0.3) (layer "F.Cu") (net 13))
 (segment (start 66.9125 84) (end 69.42 84) (width 0.3) (layer "F.Cu") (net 13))
 (segment (start 69.42 84) (end 70.5 85.08) (width 0.3) (layer "F.Cu") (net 13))
 (via (at 95.43 91.57) (size 0.9) (drill 0.5) (layers "F.Cu" "B.Cu") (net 13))
 (segment (start 70.5 85.08) (end 69.3 86.28) (width 0.3) (layer "B.Cu") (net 13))
 (segment (start 69.3 86.28) (end 69.3 88.117057) (width 0.3) (layer "B.Cu") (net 13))
 (segment (start 92.68 88.82) (end 95.43 91.57) (width 0.3) (layer "B.Cu") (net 13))
 (segment (start 70.002943 88.82) (end 92.68 88.82) (width 0.3) (layer "B.Cu") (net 13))
 (segment (start 69.3 88.117057) (end 70.002943 88.82) (width 0.3) (layer "B.Cu") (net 13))
 (segment (start 93.5 101) (end 93.5 98.75) (width 0.3) (layer "F.Cu") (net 11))
 (segment (start 95 102.5) (end 93.5 101) (width 0.3) (layer "F.Cu") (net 11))
 (segment (start 99.125 102.5) (end 95 102.5) (width 0.3) (layer "F.Cu") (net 11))
 (segment (start 93.5 98.75) (end 88.36 93.61) (width 0.3) (layer "F.Cu") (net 11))
 (segment (start 87.43 91.57) (end 84.7175 91.57) (width 0.3) (layer "F.Cu") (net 11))
 (segment (start 88.36 92.5) (end 87.43 91.57) (width 0.3) (layer "F.Cu") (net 11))
 (segment (start 88.36 93.61) (end 88.36 92.5) (width 0.3) (layer "F.Cu") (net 11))
 (segment (start 100.95 102.5) (end 104.625 102.5) (width 0.3) (layer "F.Cu") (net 21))
 (segment (start 100.95 97.5) (end 104.625 97.5) (width 0.3) (layer "F.Cu") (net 20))
 (segment (start 86.47 89.03) (end 84.7175 89.03) (width 0.3) (layer "F.Cu") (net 10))
 (segment (start 99.125 97.5) (end 97 97.5) (width 0.3) (layer "F.Cu") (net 10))
 (segment (start 97 97.5) (end 95 95.5) (width 0.3) (layer "F.Cu") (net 10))
 (segment (start 95 93) (end 94.96 92.96) (width 0.3) (layer "F.Cu") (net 10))
 (segment (start 94.96 92.96) (end 90.46 92.96) (width 0.3) (layer "F.Cu") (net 10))
 (segment (start 90.46 92.96) (end 86.5 89) (width 0.3) (layer "F.Cu") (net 10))
 (segment (start 95 95.5) (end 95 93) (width 0.3) (layer "F.Cu") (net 10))
 (segment (start 86.5 89) (end 86.47 89.03) (width 0.3) (layer "F.Cu") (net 10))
 (segment (start 97 90.18) (end 90.18 90.18) (width 0.3) (layer "F.Cu") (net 9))
 (segment (start 97 91.5) (end 97 90.18) (width 0.3) (layer "F.Cu") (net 9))
 (segment (start 86.49 86.49) (end 84.7175 86.49) (width 0.3) (layer "F.Cu") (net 9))
 (segment (start 99.2125 92.5) (end 98 92.5) (width 0.3) (layer "F.Cu") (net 9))
 (segment (start 98 92.5) (end 97 91.5) (width 0.3) (layer "F.Cu") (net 9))
 (segment (start 90.18 90.18) (end 86.49 86.49) (width 0.3) (layer "F.Cu") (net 9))
 (segment (start 101.0375 92.5) (end 104.625 92.5) (width 0.3) (layer "F.Cu") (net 22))
 (segment (start 100.95 87.5) (end 104.625 87.5) (width 0.3) (layer "F.Cu") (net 24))
 (segment (start 90.14 87.64) (end 86.45 83.95) (width 0.3) (layer "F.Cu") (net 8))
 (segment (start 86.45 83.95) (end 84.7175 83.95) (width 0.3) (layer "F.Cu") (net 8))
 (segment (start 99.125 87.5) (end 98.985 87.64) (width 0.3) (layer "F.Cu") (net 8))
 (segment (start 98.985 87.64) (end 90.14 87.64) (width 0.3) (layer "F.Cu") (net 8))
 (segment (start 100.9125 67.5) (end 104.625 67.5) (width 0.3) (layer "F.Cu") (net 19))
 (segment (start 95.5 67.5) (end 99.0875 67.5) (width 0.3) (layer "F.Cu") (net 18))
 (segment (start 92.3375 78.87) (end 93.63 78.87) (width 0.3) (layer "F.Cu") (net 18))
 (segment (start 94.5 68.5) (end 95.5 67.5) (width 0.3) (layer "F.Cu") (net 18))
 (segment (start 94.5 78) (end 94.5 68.5) (width 0.3) (layer "F.Cu") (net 18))
 (segment (start 93.63 78.87) (end 94.5 78) (width 0.3) (layer "F.Cu") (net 18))
 (segment (start 100.95 72.5) (end 104.625 72.5) (width 0.3) (layer "F.Cu") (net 4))
 (segment (start 95 73) (end 95 78.5) (width 0.3) (layer "F.Cu") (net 3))
 (segment (start 86.83 76.33) (end 84.7175 76.33) (width 0.3) (layer "F.Cu") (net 3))
 (segment (start 95.5 72.5) (end 95 73) (width 0.3) (layer "F.Cu") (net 3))
 (segment (start 93.48 80.02) (end 90.52 80.02) (width 0.3) (layer "F.Cu") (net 3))
 (segment (start 99.125 72.5) (end 95.5 72.5) (width 0.3) (layer "F.Cu") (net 3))
 (segment (start 95 78.5) (end 93.48 80.02) (width 0.3) (layer "F.Cu") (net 3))
 (segment (start 90.52 80.02) (end 86.83 76.33) (width 0.3) (layer "F.Cu") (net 3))
 (segment (start 96 81) (end 94.44 82.56) (width 0.3) (layer "F.Cu") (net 7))
 (segment (start 97 77.5) (end 96 78.5) (width 0.3) (layer "F.Cu") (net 7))
 (segment (start 94.44 82.56) (end 90.06 82.56) (width 0.3) (layer "F.Cu") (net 7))
 (segment (start 99.125 77.5) (end 97 77.5) (width 0.3) (layer "F.Cu") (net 7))
 (segment (start 84.8475 79) (end 84.7175 78.87) (width 0.3) (layer "F.Cu") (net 7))
 (segment (start 86.5 79) (end 84.8475 79) (width 0.3) (layer "F.Cu") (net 7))
 (segment (start 96 78.5) (end 96 81) (width 0.3) (layer "F.Cu") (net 7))
 (segment (start 90.06 82.56) (end 86.5 79) (width 0.3) (layer "F.Cu") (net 7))
 (segment (start 100.95 77.5) (end 104.625 77.5) (width 0.3) (layer "F.Cu") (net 23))
 (segment (start 86.41 81.41) (end 84.7175 81.41) (width 0.3) (layer "F.Cu") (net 5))
 (segment (start 96 82.5) (end 93.16 85.34) (width 0.3) (layer "F.Cu") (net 5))
 (segment (start 99.125 82.5) (end 96 82.5) (width 0.3) (layer "F.Cu") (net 5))
 (segment (start 90.34 85.34) (end 93.16 85.34) (width 0.3) (layer "F.Cu") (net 5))
 (segment (start 90.34 85.34) (end 86.41 81.41) (width 0.3) (layer "F.Cu") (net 5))
 (segment (start 100.95 82.5) (end 104.625 82.5) (width 0.3) (layer "F.Cu") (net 6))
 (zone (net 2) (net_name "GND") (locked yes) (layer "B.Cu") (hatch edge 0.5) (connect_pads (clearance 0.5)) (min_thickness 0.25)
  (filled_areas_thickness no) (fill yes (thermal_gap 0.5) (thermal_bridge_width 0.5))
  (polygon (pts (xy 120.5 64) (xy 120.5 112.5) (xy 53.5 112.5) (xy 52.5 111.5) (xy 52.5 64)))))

